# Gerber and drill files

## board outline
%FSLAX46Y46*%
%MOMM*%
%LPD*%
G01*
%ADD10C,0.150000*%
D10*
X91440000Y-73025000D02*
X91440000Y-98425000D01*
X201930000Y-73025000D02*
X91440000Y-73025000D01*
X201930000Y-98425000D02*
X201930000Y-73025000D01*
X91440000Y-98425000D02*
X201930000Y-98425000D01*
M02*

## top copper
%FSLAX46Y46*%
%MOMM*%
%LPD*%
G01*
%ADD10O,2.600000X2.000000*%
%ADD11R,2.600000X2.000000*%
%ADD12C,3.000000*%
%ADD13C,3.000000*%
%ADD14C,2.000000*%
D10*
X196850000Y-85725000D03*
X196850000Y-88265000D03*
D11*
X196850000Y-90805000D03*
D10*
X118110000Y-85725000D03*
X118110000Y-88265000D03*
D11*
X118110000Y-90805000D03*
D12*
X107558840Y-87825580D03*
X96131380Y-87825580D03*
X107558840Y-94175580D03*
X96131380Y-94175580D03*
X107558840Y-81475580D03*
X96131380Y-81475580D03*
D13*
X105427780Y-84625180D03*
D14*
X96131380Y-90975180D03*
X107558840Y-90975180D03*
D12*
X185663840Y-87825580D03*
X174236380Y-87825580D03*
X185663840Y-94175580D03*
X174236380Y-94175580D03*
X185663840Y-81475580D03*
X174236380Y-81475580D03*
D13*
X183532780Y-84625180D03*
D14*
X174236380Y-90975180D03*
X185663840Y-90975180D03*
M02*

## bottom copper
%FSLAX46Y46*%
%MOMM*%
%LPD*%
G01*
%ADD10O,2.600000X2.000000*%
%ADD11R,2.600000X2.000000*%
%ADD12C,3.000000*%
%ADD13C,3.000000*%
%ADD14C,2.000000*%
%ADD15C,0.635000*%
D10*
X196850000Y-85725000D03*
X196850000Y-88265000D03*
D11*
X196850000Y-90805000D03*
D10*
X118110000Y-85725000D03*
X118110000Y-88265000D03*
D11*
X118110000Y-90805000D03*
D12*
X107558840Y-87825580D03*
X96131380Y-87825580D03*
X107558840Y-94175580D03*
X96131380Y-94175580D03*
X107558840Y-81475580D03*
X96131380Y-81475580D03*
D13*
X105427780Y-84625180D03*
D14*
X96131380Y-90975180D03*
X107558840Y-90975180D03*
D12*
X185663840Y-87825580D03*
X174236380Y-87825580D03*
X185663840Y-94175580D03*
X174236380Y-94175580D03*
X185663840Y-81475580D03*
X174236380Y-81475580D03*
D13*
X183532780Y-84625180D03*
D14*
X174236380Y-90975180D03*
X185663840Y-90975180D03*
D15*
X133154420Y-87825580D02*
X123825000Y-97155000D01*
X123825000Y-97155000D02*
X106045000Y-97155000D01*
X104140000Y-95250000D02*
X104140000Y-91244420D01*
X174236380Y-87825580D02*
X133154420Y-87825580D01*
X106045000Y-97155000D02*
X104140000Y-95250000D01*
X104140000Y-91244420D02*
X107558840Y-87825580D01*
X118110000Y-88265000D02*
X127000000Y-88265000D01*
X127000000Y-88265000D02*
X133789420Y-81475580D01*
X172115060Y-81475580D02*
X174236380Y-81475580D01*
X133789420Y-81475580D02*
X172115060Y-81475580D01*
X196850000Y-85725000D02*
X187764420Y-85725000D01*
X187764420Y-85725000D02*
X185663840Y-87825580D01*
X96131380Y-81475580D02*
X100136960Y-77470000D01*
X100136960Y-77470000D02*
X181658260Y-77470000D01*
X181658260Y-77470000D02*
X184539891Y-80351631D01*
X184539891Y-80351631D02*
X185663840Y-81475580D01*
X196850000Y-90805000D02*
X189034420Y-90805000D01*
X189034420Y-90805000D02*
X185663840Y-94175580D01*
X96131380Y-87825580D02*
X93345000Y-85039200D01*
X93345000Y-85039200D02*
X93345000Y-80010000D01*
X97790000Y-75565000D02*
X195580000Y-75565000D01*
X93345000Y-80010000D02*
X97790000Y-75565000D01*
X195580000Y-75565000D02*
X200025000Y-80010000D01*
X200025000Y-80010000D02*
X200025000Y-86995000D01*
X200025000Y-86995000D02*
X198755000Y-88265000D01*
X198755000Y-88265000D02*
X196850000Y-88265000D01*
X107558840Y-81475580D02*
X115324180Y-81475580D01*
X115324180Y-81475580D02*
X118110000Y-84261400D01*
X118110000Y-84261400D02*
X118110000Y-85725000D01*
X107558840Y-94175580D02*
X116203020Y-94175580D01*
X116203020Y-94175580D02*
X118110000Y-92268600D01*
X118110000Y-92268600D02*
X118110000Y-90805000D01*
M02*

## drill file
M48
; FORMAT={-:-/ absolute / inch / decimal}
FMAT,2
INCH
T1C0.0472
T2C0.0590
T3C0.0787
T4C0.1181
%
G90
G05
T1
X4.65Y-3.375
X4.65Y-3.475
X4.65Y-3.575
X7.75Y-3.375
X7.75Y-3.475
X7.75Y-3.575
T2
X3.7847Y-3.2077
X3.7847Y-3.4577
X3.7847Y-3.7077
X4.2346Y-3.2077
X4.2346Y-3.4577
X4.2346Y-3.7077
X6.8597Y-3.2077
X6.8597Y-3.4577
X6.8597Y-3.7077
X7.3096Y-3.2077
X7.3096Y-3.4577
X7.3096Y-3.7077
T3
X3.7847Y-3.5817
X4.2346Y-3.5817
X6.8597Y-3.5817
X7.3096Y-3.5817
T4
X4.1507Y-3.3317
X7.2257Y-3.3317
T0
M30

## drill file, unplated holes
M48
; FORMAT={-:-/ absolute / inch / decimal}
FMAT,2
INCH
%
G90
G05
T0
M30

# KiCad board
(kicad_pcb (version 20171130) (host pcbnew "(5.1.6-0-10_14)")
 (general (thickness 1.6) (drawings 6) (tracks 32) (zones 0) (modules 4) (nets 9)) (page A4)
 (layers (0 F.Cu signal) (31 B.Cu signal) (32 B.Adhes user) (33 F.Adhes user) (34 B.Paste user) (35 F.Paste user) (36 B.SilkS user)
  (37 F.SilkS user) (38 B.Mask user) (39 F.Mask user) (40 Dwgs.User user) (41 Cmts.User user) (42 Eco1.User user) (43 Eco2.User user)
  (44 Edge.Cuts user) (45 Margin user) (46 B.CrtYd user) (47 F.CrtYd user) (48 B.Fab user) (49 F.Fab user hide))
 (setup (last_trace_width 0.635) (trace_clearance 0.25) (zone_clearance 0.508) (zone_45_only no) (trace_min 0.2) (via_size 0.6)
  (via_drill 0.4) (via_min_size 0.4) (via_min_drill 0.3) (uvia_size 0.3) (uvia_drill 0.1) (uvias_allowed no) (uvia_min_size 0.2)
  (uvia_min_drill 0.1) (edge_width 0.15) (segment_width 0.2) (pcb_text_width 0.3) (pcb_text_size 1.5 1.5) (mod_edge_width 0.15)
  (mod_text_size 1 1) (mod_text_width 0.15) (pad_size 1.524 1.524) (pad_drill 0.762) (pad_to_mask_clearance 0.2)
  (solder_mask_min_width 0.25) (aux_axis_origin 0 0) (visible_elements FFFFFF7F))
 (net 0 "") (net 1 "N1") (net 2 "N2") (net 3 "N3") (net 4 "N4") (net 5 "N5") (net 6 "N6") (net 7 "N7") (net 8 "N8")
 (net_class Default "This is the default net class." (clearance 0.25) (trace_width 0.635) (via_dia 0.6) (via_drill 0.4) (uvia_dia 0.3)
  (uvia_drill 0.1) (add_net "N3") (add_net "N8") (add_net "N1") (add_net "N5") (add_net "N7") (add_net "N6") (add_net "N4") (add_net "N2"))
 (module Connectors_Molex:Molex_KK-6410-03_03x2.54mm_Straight (layer F.Cu) (at 196.85 90.805 90)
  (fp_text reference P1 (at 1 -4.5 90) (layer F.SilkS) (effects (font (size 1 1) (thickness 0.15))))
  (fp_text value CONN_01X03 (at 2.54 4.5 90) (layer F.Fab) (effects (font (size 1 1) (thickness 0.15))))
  (pad 3 thru_hole oval (at 5.08 0 90) (size 2 2.6) (drill 1.2) (layers *.Cu *.Mask) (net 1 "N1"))
  (pad 2 thru_hole oval (at 2.54 0 90) (size 2 2.6) (drill 1.2) (layers *.Cu *.Mask) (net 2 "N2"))
  (pad 1 thru_hole rect (at 0 0 90) (size 2 2.6) (drill 1.2) (layers *.Cu *.Mask) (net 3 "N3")))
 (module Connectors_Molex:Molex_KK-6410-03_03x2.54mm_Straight (layer F.Cu) (at 118.11 90.805 90)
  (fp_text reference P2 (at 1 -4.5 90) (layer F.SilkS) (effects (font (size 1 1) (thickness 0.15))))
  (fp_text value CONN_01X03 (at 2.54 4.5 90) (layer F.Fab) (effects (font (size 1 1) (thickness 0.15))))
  (pad 3 thru_hole oval (at 5.08 0 90) (size 2 2.6) (drill 1.2) (layers *.Cu *.Mask) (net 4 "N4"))
  (pad 2 thru_hole oval (at 2.54 0 90) (size 2 2.6) (drill 1.2) (layers *.Cu *.Mask) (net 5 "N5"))
  (pad 1 thru_hole rect (at 0 0 90) (size 2 2.6) (drill 1.2) (layers *.Cu *.Mask) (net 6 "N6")))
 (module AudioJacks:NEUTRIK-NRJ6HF (layer F.Cu) (at 100.33 98.425)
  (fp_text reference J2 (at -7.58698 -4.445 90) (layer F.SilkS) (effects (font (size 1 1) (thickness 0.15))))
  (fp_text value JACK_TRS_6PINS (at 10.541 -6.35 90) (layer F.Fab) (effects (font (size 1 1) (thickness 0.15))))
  (pad 3 thru_hole circle (at 7.22884 -10.59942) (size 3 3) (drill 1.4986) (layers *.Cu *.Mask F.SilkS) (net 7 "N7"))
  (pad 6 thru_hole circle (at -4.19862 -10.59942) (size 3 3) (drill 1.4986) (layers *.Cu *.Mask F.SilkS) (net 2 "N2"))
  (pad 1 thru_hole circle (at 7.22884 -4.24942) (size 3 3) (drill 1.4986) (layers *.Cu *.Mask F.SilkS) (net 6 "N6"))
  (pad 4 thru_hole circle (at -4.19862 -4.24942) (size 3 3) (drill 1.4986) (layers *.Cu *.Mask F.SilkS))
  (pad 2 thru_hole circle (at 7.22884 -16.94942) (size 3 3) (drill 1.4986) (layers *.Cu *.Mask F.SilkS) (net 4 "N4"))
  (pad 5 thru_hole circle (at -4.19862 -16.94942) (size 3 3) (drill 1.4986) (layers *.Cu *.Mask F.SilkS) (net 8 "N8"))
  (pad "" thru_hole circle (at 5.09778 -13.79982) (size 3 3) (drill 3) (layers *.Cu))
  (pad "" thru_hole circle (at -4.19862 -7.44982) (size 2 2) (drill 2) (layers *.Cu))
  (pad "" thru_hole circle (at 7.22884 -7.44982) (size 2 2) (drill 2) (layers *.Cu)))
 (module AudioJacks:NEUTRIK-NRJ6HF (layer F.Cu) (at 178.435 98.425)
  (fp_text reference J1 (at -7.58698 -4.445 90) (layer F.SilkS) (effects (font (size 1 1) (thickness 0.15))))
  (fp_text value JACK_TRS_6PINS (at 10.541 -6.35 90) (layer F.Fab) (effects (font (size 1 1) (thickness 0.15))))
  (pad 3 thru_hole circle (at 7.22884 -10.59942) (size 3 3) (drill 1.4986) (layers *.Cu *.Mask F.SilkS) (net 1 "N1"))
  (pad 6 thru_hole circle (at -4.19862 -10.59942) (size 3 3) (drill 1.4986) (layers *.Cu *.Mask F.SilkS) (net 7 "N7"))
  (pad 1 thru_hole circle (at 7.22884 -4.24942) (size 3 3) (drill 1.4986) (layers *.Cu *.Mask F.SilkS) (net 3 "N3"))
  (pad 4 thru_hole circle (at -4.19862 -4.24942) (size 3 3) (drill 1.4986) (layers *.Cu *.Mask F.SilkS))
  (pad 2 thru_hole circle (at 7.22884 -16.94942) (size 3 3) (drill 1.4986) (layers *.Cu *.Mask F.SilkS) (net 8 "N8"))
  (pad 5 thru_hole circle (at -4.19862 -16.94942) (size 3 3) (drill 1.4986) (layers *.Cu *.Mask F.SilkS) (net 5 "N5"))
  (pad "" thru_hole circle (at 5.09778 -13.79982) (size 3 3) (drill 3) (layers *.Cu))
  (pad "" thru_hole circle (at -4.19862 -7.44982) (size 2 2) (drill 2) (layers *.Cu))
  (pad "" thru_hole circle (at 7.22884 -7.44982) (size 2 2) (drill 2) (layers *.Cu)))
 (gr_line (start 91.44 73.025) (end 91.44 98.425) (layer Edge.Cuts) (width 0.15))
 (gr_line (start 201.93 73.025) (end 91.44 73.025) (layer Edge.Cuts) (width 0.15))
 (gr_line (start 201.93 98.425) (end 201.93 73.025) (layer Edge.Cuts) (width 0.15))
 (gr_line (start 91.44 98.425) (end 201.93 98.425) (layer Edge.Cuts) (width 0.15))
 (segment (start 133.15442 87.82558) (end 123.825 97.155) (width 0.635) (layer B.Cu) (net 7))
 (segment (start 123.825 97.155) (end 106.045 97.155) (width 0.635) (layer B.Cu) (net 7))
 (segment (start 104.14 95.25) (end 104.14 91.24442) (width 0.635) (layer B.Cu) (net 7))
 (segment (start 174.23638 87.82558) (end 133.15442 87.82558) (width 0.635) (layer B.Cu) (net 7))
 (segment (start 106.045 97.155) (end 104.14 95.25) (width 0.635) (layer B.Cu) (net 7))
 (segment (start 104.14 91.24442) (end 107.55884 87.82558) (width 0.635) (layer B.Cu) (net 7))
 (segment (start 118.11 88.265) (end 127 88.265) (width 0.635) (layer B.Cu) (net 5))
 (segment (start 127 88.265) (end 133.78942 81.47558) (width 0.635) (layer B.Cu) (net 5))
 (segment (start 172.11506 81.47558) (end 174.23638 81.47558) (width 0.635) (layer B.Cu) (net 5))
 (segment (start 133.78942 81.47558) (end 172.11506 81.47558) (width 0.635) (layer B.Cu) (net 5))
 (segment (start 196.85 85.725) (end 187.76442 85.725) (width 0.635) (layer B.Cu) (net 1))
 (segment (start 187.76442 85.725) (end 185.66384 87.82558) (width 0.635) (layer B.Cu) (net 1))
 (segment (start 96.13138 81.47558) (end 100.13696 77.47) (width 0.635) (layer B.Cu) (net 8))
 (segment (start 100.13696 77.47) (end 181.65826 77.47) (width 0.635) (layer B.Cu) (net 8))
 (segment (start 181.65826 77.47) (end 184.539891 80.351631) (width 0.635) (layer B.Cu) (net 8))
 (segment (start 184.539891 80.351631) (end 185.66384 81.47558) (width 0.635) (layer B.Cu) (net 8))
 (segment (start 196.85 90.805) (end 189.03442 90.805) (width 0.635) (layer B.Cu) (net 3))
 (segment (start 189.03442 90.805) (end 185.66384 94.17558) (width 0.635) (layer B.Cu) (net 3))
 (segment (start 96.13138 87.82558) (end 93.345 85.0392) (width 0.635) (layer B.Cu) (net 2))
 (segment (start 93.345 85.0392) (end 93.345 80.01) (width 0.635) (layer B.Cu) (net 2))
 (segment (start 97.79 75.565) (end 195.58 75.565) (width 0.635) (layer B.Cu) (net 2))
 (segment (start 93.345 80.01) (end 97.79 75.565) (width 0.635) (layer B.Cu) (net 2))
 (segment (start 195.58 75.565) (end 200.025 80.01) (width 0.635) (layer B.Cu) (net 2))
 (segment (start 200.025 80.01) (end 200.025 86.995) (width 0.635) (layer B.Cu) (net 2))
 (segment (start 200.025 86.995) (end 198.755 88.265) (width 0.635) (layer B.Cu) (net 2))
 (segment (start 198.755 88.265) (end 196.85 88.265) (width 0.635) (layer B.Cu) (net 2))
 (segment (start 107.55884 81.47558) (end 115.32418 81.47558) (width 0.635) (layer B.Cu) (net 4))
 (segment (start 115.32418 81.47558) (end 118.11 84.2614) (width 0.635) (layer B.Cu) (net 4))
 (segment (start 118.11 84.2614) (end 118.11 85.725) (width 0.635) (layer B.Cu) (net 4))
 (segment (start 107.55884 94.17558) (end 116.20302 94.17558) (width 0.635) (layer B.Cu) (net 6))
 (segment (start 116.20302 94.17558) (end 118.11 92.2686) (width 0.635) (layer B.Cu) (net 6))
 (segment (start 118.11 92.2686) (end 118.11 90.805) (width 0.635) (layer B.Cu) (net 6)))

